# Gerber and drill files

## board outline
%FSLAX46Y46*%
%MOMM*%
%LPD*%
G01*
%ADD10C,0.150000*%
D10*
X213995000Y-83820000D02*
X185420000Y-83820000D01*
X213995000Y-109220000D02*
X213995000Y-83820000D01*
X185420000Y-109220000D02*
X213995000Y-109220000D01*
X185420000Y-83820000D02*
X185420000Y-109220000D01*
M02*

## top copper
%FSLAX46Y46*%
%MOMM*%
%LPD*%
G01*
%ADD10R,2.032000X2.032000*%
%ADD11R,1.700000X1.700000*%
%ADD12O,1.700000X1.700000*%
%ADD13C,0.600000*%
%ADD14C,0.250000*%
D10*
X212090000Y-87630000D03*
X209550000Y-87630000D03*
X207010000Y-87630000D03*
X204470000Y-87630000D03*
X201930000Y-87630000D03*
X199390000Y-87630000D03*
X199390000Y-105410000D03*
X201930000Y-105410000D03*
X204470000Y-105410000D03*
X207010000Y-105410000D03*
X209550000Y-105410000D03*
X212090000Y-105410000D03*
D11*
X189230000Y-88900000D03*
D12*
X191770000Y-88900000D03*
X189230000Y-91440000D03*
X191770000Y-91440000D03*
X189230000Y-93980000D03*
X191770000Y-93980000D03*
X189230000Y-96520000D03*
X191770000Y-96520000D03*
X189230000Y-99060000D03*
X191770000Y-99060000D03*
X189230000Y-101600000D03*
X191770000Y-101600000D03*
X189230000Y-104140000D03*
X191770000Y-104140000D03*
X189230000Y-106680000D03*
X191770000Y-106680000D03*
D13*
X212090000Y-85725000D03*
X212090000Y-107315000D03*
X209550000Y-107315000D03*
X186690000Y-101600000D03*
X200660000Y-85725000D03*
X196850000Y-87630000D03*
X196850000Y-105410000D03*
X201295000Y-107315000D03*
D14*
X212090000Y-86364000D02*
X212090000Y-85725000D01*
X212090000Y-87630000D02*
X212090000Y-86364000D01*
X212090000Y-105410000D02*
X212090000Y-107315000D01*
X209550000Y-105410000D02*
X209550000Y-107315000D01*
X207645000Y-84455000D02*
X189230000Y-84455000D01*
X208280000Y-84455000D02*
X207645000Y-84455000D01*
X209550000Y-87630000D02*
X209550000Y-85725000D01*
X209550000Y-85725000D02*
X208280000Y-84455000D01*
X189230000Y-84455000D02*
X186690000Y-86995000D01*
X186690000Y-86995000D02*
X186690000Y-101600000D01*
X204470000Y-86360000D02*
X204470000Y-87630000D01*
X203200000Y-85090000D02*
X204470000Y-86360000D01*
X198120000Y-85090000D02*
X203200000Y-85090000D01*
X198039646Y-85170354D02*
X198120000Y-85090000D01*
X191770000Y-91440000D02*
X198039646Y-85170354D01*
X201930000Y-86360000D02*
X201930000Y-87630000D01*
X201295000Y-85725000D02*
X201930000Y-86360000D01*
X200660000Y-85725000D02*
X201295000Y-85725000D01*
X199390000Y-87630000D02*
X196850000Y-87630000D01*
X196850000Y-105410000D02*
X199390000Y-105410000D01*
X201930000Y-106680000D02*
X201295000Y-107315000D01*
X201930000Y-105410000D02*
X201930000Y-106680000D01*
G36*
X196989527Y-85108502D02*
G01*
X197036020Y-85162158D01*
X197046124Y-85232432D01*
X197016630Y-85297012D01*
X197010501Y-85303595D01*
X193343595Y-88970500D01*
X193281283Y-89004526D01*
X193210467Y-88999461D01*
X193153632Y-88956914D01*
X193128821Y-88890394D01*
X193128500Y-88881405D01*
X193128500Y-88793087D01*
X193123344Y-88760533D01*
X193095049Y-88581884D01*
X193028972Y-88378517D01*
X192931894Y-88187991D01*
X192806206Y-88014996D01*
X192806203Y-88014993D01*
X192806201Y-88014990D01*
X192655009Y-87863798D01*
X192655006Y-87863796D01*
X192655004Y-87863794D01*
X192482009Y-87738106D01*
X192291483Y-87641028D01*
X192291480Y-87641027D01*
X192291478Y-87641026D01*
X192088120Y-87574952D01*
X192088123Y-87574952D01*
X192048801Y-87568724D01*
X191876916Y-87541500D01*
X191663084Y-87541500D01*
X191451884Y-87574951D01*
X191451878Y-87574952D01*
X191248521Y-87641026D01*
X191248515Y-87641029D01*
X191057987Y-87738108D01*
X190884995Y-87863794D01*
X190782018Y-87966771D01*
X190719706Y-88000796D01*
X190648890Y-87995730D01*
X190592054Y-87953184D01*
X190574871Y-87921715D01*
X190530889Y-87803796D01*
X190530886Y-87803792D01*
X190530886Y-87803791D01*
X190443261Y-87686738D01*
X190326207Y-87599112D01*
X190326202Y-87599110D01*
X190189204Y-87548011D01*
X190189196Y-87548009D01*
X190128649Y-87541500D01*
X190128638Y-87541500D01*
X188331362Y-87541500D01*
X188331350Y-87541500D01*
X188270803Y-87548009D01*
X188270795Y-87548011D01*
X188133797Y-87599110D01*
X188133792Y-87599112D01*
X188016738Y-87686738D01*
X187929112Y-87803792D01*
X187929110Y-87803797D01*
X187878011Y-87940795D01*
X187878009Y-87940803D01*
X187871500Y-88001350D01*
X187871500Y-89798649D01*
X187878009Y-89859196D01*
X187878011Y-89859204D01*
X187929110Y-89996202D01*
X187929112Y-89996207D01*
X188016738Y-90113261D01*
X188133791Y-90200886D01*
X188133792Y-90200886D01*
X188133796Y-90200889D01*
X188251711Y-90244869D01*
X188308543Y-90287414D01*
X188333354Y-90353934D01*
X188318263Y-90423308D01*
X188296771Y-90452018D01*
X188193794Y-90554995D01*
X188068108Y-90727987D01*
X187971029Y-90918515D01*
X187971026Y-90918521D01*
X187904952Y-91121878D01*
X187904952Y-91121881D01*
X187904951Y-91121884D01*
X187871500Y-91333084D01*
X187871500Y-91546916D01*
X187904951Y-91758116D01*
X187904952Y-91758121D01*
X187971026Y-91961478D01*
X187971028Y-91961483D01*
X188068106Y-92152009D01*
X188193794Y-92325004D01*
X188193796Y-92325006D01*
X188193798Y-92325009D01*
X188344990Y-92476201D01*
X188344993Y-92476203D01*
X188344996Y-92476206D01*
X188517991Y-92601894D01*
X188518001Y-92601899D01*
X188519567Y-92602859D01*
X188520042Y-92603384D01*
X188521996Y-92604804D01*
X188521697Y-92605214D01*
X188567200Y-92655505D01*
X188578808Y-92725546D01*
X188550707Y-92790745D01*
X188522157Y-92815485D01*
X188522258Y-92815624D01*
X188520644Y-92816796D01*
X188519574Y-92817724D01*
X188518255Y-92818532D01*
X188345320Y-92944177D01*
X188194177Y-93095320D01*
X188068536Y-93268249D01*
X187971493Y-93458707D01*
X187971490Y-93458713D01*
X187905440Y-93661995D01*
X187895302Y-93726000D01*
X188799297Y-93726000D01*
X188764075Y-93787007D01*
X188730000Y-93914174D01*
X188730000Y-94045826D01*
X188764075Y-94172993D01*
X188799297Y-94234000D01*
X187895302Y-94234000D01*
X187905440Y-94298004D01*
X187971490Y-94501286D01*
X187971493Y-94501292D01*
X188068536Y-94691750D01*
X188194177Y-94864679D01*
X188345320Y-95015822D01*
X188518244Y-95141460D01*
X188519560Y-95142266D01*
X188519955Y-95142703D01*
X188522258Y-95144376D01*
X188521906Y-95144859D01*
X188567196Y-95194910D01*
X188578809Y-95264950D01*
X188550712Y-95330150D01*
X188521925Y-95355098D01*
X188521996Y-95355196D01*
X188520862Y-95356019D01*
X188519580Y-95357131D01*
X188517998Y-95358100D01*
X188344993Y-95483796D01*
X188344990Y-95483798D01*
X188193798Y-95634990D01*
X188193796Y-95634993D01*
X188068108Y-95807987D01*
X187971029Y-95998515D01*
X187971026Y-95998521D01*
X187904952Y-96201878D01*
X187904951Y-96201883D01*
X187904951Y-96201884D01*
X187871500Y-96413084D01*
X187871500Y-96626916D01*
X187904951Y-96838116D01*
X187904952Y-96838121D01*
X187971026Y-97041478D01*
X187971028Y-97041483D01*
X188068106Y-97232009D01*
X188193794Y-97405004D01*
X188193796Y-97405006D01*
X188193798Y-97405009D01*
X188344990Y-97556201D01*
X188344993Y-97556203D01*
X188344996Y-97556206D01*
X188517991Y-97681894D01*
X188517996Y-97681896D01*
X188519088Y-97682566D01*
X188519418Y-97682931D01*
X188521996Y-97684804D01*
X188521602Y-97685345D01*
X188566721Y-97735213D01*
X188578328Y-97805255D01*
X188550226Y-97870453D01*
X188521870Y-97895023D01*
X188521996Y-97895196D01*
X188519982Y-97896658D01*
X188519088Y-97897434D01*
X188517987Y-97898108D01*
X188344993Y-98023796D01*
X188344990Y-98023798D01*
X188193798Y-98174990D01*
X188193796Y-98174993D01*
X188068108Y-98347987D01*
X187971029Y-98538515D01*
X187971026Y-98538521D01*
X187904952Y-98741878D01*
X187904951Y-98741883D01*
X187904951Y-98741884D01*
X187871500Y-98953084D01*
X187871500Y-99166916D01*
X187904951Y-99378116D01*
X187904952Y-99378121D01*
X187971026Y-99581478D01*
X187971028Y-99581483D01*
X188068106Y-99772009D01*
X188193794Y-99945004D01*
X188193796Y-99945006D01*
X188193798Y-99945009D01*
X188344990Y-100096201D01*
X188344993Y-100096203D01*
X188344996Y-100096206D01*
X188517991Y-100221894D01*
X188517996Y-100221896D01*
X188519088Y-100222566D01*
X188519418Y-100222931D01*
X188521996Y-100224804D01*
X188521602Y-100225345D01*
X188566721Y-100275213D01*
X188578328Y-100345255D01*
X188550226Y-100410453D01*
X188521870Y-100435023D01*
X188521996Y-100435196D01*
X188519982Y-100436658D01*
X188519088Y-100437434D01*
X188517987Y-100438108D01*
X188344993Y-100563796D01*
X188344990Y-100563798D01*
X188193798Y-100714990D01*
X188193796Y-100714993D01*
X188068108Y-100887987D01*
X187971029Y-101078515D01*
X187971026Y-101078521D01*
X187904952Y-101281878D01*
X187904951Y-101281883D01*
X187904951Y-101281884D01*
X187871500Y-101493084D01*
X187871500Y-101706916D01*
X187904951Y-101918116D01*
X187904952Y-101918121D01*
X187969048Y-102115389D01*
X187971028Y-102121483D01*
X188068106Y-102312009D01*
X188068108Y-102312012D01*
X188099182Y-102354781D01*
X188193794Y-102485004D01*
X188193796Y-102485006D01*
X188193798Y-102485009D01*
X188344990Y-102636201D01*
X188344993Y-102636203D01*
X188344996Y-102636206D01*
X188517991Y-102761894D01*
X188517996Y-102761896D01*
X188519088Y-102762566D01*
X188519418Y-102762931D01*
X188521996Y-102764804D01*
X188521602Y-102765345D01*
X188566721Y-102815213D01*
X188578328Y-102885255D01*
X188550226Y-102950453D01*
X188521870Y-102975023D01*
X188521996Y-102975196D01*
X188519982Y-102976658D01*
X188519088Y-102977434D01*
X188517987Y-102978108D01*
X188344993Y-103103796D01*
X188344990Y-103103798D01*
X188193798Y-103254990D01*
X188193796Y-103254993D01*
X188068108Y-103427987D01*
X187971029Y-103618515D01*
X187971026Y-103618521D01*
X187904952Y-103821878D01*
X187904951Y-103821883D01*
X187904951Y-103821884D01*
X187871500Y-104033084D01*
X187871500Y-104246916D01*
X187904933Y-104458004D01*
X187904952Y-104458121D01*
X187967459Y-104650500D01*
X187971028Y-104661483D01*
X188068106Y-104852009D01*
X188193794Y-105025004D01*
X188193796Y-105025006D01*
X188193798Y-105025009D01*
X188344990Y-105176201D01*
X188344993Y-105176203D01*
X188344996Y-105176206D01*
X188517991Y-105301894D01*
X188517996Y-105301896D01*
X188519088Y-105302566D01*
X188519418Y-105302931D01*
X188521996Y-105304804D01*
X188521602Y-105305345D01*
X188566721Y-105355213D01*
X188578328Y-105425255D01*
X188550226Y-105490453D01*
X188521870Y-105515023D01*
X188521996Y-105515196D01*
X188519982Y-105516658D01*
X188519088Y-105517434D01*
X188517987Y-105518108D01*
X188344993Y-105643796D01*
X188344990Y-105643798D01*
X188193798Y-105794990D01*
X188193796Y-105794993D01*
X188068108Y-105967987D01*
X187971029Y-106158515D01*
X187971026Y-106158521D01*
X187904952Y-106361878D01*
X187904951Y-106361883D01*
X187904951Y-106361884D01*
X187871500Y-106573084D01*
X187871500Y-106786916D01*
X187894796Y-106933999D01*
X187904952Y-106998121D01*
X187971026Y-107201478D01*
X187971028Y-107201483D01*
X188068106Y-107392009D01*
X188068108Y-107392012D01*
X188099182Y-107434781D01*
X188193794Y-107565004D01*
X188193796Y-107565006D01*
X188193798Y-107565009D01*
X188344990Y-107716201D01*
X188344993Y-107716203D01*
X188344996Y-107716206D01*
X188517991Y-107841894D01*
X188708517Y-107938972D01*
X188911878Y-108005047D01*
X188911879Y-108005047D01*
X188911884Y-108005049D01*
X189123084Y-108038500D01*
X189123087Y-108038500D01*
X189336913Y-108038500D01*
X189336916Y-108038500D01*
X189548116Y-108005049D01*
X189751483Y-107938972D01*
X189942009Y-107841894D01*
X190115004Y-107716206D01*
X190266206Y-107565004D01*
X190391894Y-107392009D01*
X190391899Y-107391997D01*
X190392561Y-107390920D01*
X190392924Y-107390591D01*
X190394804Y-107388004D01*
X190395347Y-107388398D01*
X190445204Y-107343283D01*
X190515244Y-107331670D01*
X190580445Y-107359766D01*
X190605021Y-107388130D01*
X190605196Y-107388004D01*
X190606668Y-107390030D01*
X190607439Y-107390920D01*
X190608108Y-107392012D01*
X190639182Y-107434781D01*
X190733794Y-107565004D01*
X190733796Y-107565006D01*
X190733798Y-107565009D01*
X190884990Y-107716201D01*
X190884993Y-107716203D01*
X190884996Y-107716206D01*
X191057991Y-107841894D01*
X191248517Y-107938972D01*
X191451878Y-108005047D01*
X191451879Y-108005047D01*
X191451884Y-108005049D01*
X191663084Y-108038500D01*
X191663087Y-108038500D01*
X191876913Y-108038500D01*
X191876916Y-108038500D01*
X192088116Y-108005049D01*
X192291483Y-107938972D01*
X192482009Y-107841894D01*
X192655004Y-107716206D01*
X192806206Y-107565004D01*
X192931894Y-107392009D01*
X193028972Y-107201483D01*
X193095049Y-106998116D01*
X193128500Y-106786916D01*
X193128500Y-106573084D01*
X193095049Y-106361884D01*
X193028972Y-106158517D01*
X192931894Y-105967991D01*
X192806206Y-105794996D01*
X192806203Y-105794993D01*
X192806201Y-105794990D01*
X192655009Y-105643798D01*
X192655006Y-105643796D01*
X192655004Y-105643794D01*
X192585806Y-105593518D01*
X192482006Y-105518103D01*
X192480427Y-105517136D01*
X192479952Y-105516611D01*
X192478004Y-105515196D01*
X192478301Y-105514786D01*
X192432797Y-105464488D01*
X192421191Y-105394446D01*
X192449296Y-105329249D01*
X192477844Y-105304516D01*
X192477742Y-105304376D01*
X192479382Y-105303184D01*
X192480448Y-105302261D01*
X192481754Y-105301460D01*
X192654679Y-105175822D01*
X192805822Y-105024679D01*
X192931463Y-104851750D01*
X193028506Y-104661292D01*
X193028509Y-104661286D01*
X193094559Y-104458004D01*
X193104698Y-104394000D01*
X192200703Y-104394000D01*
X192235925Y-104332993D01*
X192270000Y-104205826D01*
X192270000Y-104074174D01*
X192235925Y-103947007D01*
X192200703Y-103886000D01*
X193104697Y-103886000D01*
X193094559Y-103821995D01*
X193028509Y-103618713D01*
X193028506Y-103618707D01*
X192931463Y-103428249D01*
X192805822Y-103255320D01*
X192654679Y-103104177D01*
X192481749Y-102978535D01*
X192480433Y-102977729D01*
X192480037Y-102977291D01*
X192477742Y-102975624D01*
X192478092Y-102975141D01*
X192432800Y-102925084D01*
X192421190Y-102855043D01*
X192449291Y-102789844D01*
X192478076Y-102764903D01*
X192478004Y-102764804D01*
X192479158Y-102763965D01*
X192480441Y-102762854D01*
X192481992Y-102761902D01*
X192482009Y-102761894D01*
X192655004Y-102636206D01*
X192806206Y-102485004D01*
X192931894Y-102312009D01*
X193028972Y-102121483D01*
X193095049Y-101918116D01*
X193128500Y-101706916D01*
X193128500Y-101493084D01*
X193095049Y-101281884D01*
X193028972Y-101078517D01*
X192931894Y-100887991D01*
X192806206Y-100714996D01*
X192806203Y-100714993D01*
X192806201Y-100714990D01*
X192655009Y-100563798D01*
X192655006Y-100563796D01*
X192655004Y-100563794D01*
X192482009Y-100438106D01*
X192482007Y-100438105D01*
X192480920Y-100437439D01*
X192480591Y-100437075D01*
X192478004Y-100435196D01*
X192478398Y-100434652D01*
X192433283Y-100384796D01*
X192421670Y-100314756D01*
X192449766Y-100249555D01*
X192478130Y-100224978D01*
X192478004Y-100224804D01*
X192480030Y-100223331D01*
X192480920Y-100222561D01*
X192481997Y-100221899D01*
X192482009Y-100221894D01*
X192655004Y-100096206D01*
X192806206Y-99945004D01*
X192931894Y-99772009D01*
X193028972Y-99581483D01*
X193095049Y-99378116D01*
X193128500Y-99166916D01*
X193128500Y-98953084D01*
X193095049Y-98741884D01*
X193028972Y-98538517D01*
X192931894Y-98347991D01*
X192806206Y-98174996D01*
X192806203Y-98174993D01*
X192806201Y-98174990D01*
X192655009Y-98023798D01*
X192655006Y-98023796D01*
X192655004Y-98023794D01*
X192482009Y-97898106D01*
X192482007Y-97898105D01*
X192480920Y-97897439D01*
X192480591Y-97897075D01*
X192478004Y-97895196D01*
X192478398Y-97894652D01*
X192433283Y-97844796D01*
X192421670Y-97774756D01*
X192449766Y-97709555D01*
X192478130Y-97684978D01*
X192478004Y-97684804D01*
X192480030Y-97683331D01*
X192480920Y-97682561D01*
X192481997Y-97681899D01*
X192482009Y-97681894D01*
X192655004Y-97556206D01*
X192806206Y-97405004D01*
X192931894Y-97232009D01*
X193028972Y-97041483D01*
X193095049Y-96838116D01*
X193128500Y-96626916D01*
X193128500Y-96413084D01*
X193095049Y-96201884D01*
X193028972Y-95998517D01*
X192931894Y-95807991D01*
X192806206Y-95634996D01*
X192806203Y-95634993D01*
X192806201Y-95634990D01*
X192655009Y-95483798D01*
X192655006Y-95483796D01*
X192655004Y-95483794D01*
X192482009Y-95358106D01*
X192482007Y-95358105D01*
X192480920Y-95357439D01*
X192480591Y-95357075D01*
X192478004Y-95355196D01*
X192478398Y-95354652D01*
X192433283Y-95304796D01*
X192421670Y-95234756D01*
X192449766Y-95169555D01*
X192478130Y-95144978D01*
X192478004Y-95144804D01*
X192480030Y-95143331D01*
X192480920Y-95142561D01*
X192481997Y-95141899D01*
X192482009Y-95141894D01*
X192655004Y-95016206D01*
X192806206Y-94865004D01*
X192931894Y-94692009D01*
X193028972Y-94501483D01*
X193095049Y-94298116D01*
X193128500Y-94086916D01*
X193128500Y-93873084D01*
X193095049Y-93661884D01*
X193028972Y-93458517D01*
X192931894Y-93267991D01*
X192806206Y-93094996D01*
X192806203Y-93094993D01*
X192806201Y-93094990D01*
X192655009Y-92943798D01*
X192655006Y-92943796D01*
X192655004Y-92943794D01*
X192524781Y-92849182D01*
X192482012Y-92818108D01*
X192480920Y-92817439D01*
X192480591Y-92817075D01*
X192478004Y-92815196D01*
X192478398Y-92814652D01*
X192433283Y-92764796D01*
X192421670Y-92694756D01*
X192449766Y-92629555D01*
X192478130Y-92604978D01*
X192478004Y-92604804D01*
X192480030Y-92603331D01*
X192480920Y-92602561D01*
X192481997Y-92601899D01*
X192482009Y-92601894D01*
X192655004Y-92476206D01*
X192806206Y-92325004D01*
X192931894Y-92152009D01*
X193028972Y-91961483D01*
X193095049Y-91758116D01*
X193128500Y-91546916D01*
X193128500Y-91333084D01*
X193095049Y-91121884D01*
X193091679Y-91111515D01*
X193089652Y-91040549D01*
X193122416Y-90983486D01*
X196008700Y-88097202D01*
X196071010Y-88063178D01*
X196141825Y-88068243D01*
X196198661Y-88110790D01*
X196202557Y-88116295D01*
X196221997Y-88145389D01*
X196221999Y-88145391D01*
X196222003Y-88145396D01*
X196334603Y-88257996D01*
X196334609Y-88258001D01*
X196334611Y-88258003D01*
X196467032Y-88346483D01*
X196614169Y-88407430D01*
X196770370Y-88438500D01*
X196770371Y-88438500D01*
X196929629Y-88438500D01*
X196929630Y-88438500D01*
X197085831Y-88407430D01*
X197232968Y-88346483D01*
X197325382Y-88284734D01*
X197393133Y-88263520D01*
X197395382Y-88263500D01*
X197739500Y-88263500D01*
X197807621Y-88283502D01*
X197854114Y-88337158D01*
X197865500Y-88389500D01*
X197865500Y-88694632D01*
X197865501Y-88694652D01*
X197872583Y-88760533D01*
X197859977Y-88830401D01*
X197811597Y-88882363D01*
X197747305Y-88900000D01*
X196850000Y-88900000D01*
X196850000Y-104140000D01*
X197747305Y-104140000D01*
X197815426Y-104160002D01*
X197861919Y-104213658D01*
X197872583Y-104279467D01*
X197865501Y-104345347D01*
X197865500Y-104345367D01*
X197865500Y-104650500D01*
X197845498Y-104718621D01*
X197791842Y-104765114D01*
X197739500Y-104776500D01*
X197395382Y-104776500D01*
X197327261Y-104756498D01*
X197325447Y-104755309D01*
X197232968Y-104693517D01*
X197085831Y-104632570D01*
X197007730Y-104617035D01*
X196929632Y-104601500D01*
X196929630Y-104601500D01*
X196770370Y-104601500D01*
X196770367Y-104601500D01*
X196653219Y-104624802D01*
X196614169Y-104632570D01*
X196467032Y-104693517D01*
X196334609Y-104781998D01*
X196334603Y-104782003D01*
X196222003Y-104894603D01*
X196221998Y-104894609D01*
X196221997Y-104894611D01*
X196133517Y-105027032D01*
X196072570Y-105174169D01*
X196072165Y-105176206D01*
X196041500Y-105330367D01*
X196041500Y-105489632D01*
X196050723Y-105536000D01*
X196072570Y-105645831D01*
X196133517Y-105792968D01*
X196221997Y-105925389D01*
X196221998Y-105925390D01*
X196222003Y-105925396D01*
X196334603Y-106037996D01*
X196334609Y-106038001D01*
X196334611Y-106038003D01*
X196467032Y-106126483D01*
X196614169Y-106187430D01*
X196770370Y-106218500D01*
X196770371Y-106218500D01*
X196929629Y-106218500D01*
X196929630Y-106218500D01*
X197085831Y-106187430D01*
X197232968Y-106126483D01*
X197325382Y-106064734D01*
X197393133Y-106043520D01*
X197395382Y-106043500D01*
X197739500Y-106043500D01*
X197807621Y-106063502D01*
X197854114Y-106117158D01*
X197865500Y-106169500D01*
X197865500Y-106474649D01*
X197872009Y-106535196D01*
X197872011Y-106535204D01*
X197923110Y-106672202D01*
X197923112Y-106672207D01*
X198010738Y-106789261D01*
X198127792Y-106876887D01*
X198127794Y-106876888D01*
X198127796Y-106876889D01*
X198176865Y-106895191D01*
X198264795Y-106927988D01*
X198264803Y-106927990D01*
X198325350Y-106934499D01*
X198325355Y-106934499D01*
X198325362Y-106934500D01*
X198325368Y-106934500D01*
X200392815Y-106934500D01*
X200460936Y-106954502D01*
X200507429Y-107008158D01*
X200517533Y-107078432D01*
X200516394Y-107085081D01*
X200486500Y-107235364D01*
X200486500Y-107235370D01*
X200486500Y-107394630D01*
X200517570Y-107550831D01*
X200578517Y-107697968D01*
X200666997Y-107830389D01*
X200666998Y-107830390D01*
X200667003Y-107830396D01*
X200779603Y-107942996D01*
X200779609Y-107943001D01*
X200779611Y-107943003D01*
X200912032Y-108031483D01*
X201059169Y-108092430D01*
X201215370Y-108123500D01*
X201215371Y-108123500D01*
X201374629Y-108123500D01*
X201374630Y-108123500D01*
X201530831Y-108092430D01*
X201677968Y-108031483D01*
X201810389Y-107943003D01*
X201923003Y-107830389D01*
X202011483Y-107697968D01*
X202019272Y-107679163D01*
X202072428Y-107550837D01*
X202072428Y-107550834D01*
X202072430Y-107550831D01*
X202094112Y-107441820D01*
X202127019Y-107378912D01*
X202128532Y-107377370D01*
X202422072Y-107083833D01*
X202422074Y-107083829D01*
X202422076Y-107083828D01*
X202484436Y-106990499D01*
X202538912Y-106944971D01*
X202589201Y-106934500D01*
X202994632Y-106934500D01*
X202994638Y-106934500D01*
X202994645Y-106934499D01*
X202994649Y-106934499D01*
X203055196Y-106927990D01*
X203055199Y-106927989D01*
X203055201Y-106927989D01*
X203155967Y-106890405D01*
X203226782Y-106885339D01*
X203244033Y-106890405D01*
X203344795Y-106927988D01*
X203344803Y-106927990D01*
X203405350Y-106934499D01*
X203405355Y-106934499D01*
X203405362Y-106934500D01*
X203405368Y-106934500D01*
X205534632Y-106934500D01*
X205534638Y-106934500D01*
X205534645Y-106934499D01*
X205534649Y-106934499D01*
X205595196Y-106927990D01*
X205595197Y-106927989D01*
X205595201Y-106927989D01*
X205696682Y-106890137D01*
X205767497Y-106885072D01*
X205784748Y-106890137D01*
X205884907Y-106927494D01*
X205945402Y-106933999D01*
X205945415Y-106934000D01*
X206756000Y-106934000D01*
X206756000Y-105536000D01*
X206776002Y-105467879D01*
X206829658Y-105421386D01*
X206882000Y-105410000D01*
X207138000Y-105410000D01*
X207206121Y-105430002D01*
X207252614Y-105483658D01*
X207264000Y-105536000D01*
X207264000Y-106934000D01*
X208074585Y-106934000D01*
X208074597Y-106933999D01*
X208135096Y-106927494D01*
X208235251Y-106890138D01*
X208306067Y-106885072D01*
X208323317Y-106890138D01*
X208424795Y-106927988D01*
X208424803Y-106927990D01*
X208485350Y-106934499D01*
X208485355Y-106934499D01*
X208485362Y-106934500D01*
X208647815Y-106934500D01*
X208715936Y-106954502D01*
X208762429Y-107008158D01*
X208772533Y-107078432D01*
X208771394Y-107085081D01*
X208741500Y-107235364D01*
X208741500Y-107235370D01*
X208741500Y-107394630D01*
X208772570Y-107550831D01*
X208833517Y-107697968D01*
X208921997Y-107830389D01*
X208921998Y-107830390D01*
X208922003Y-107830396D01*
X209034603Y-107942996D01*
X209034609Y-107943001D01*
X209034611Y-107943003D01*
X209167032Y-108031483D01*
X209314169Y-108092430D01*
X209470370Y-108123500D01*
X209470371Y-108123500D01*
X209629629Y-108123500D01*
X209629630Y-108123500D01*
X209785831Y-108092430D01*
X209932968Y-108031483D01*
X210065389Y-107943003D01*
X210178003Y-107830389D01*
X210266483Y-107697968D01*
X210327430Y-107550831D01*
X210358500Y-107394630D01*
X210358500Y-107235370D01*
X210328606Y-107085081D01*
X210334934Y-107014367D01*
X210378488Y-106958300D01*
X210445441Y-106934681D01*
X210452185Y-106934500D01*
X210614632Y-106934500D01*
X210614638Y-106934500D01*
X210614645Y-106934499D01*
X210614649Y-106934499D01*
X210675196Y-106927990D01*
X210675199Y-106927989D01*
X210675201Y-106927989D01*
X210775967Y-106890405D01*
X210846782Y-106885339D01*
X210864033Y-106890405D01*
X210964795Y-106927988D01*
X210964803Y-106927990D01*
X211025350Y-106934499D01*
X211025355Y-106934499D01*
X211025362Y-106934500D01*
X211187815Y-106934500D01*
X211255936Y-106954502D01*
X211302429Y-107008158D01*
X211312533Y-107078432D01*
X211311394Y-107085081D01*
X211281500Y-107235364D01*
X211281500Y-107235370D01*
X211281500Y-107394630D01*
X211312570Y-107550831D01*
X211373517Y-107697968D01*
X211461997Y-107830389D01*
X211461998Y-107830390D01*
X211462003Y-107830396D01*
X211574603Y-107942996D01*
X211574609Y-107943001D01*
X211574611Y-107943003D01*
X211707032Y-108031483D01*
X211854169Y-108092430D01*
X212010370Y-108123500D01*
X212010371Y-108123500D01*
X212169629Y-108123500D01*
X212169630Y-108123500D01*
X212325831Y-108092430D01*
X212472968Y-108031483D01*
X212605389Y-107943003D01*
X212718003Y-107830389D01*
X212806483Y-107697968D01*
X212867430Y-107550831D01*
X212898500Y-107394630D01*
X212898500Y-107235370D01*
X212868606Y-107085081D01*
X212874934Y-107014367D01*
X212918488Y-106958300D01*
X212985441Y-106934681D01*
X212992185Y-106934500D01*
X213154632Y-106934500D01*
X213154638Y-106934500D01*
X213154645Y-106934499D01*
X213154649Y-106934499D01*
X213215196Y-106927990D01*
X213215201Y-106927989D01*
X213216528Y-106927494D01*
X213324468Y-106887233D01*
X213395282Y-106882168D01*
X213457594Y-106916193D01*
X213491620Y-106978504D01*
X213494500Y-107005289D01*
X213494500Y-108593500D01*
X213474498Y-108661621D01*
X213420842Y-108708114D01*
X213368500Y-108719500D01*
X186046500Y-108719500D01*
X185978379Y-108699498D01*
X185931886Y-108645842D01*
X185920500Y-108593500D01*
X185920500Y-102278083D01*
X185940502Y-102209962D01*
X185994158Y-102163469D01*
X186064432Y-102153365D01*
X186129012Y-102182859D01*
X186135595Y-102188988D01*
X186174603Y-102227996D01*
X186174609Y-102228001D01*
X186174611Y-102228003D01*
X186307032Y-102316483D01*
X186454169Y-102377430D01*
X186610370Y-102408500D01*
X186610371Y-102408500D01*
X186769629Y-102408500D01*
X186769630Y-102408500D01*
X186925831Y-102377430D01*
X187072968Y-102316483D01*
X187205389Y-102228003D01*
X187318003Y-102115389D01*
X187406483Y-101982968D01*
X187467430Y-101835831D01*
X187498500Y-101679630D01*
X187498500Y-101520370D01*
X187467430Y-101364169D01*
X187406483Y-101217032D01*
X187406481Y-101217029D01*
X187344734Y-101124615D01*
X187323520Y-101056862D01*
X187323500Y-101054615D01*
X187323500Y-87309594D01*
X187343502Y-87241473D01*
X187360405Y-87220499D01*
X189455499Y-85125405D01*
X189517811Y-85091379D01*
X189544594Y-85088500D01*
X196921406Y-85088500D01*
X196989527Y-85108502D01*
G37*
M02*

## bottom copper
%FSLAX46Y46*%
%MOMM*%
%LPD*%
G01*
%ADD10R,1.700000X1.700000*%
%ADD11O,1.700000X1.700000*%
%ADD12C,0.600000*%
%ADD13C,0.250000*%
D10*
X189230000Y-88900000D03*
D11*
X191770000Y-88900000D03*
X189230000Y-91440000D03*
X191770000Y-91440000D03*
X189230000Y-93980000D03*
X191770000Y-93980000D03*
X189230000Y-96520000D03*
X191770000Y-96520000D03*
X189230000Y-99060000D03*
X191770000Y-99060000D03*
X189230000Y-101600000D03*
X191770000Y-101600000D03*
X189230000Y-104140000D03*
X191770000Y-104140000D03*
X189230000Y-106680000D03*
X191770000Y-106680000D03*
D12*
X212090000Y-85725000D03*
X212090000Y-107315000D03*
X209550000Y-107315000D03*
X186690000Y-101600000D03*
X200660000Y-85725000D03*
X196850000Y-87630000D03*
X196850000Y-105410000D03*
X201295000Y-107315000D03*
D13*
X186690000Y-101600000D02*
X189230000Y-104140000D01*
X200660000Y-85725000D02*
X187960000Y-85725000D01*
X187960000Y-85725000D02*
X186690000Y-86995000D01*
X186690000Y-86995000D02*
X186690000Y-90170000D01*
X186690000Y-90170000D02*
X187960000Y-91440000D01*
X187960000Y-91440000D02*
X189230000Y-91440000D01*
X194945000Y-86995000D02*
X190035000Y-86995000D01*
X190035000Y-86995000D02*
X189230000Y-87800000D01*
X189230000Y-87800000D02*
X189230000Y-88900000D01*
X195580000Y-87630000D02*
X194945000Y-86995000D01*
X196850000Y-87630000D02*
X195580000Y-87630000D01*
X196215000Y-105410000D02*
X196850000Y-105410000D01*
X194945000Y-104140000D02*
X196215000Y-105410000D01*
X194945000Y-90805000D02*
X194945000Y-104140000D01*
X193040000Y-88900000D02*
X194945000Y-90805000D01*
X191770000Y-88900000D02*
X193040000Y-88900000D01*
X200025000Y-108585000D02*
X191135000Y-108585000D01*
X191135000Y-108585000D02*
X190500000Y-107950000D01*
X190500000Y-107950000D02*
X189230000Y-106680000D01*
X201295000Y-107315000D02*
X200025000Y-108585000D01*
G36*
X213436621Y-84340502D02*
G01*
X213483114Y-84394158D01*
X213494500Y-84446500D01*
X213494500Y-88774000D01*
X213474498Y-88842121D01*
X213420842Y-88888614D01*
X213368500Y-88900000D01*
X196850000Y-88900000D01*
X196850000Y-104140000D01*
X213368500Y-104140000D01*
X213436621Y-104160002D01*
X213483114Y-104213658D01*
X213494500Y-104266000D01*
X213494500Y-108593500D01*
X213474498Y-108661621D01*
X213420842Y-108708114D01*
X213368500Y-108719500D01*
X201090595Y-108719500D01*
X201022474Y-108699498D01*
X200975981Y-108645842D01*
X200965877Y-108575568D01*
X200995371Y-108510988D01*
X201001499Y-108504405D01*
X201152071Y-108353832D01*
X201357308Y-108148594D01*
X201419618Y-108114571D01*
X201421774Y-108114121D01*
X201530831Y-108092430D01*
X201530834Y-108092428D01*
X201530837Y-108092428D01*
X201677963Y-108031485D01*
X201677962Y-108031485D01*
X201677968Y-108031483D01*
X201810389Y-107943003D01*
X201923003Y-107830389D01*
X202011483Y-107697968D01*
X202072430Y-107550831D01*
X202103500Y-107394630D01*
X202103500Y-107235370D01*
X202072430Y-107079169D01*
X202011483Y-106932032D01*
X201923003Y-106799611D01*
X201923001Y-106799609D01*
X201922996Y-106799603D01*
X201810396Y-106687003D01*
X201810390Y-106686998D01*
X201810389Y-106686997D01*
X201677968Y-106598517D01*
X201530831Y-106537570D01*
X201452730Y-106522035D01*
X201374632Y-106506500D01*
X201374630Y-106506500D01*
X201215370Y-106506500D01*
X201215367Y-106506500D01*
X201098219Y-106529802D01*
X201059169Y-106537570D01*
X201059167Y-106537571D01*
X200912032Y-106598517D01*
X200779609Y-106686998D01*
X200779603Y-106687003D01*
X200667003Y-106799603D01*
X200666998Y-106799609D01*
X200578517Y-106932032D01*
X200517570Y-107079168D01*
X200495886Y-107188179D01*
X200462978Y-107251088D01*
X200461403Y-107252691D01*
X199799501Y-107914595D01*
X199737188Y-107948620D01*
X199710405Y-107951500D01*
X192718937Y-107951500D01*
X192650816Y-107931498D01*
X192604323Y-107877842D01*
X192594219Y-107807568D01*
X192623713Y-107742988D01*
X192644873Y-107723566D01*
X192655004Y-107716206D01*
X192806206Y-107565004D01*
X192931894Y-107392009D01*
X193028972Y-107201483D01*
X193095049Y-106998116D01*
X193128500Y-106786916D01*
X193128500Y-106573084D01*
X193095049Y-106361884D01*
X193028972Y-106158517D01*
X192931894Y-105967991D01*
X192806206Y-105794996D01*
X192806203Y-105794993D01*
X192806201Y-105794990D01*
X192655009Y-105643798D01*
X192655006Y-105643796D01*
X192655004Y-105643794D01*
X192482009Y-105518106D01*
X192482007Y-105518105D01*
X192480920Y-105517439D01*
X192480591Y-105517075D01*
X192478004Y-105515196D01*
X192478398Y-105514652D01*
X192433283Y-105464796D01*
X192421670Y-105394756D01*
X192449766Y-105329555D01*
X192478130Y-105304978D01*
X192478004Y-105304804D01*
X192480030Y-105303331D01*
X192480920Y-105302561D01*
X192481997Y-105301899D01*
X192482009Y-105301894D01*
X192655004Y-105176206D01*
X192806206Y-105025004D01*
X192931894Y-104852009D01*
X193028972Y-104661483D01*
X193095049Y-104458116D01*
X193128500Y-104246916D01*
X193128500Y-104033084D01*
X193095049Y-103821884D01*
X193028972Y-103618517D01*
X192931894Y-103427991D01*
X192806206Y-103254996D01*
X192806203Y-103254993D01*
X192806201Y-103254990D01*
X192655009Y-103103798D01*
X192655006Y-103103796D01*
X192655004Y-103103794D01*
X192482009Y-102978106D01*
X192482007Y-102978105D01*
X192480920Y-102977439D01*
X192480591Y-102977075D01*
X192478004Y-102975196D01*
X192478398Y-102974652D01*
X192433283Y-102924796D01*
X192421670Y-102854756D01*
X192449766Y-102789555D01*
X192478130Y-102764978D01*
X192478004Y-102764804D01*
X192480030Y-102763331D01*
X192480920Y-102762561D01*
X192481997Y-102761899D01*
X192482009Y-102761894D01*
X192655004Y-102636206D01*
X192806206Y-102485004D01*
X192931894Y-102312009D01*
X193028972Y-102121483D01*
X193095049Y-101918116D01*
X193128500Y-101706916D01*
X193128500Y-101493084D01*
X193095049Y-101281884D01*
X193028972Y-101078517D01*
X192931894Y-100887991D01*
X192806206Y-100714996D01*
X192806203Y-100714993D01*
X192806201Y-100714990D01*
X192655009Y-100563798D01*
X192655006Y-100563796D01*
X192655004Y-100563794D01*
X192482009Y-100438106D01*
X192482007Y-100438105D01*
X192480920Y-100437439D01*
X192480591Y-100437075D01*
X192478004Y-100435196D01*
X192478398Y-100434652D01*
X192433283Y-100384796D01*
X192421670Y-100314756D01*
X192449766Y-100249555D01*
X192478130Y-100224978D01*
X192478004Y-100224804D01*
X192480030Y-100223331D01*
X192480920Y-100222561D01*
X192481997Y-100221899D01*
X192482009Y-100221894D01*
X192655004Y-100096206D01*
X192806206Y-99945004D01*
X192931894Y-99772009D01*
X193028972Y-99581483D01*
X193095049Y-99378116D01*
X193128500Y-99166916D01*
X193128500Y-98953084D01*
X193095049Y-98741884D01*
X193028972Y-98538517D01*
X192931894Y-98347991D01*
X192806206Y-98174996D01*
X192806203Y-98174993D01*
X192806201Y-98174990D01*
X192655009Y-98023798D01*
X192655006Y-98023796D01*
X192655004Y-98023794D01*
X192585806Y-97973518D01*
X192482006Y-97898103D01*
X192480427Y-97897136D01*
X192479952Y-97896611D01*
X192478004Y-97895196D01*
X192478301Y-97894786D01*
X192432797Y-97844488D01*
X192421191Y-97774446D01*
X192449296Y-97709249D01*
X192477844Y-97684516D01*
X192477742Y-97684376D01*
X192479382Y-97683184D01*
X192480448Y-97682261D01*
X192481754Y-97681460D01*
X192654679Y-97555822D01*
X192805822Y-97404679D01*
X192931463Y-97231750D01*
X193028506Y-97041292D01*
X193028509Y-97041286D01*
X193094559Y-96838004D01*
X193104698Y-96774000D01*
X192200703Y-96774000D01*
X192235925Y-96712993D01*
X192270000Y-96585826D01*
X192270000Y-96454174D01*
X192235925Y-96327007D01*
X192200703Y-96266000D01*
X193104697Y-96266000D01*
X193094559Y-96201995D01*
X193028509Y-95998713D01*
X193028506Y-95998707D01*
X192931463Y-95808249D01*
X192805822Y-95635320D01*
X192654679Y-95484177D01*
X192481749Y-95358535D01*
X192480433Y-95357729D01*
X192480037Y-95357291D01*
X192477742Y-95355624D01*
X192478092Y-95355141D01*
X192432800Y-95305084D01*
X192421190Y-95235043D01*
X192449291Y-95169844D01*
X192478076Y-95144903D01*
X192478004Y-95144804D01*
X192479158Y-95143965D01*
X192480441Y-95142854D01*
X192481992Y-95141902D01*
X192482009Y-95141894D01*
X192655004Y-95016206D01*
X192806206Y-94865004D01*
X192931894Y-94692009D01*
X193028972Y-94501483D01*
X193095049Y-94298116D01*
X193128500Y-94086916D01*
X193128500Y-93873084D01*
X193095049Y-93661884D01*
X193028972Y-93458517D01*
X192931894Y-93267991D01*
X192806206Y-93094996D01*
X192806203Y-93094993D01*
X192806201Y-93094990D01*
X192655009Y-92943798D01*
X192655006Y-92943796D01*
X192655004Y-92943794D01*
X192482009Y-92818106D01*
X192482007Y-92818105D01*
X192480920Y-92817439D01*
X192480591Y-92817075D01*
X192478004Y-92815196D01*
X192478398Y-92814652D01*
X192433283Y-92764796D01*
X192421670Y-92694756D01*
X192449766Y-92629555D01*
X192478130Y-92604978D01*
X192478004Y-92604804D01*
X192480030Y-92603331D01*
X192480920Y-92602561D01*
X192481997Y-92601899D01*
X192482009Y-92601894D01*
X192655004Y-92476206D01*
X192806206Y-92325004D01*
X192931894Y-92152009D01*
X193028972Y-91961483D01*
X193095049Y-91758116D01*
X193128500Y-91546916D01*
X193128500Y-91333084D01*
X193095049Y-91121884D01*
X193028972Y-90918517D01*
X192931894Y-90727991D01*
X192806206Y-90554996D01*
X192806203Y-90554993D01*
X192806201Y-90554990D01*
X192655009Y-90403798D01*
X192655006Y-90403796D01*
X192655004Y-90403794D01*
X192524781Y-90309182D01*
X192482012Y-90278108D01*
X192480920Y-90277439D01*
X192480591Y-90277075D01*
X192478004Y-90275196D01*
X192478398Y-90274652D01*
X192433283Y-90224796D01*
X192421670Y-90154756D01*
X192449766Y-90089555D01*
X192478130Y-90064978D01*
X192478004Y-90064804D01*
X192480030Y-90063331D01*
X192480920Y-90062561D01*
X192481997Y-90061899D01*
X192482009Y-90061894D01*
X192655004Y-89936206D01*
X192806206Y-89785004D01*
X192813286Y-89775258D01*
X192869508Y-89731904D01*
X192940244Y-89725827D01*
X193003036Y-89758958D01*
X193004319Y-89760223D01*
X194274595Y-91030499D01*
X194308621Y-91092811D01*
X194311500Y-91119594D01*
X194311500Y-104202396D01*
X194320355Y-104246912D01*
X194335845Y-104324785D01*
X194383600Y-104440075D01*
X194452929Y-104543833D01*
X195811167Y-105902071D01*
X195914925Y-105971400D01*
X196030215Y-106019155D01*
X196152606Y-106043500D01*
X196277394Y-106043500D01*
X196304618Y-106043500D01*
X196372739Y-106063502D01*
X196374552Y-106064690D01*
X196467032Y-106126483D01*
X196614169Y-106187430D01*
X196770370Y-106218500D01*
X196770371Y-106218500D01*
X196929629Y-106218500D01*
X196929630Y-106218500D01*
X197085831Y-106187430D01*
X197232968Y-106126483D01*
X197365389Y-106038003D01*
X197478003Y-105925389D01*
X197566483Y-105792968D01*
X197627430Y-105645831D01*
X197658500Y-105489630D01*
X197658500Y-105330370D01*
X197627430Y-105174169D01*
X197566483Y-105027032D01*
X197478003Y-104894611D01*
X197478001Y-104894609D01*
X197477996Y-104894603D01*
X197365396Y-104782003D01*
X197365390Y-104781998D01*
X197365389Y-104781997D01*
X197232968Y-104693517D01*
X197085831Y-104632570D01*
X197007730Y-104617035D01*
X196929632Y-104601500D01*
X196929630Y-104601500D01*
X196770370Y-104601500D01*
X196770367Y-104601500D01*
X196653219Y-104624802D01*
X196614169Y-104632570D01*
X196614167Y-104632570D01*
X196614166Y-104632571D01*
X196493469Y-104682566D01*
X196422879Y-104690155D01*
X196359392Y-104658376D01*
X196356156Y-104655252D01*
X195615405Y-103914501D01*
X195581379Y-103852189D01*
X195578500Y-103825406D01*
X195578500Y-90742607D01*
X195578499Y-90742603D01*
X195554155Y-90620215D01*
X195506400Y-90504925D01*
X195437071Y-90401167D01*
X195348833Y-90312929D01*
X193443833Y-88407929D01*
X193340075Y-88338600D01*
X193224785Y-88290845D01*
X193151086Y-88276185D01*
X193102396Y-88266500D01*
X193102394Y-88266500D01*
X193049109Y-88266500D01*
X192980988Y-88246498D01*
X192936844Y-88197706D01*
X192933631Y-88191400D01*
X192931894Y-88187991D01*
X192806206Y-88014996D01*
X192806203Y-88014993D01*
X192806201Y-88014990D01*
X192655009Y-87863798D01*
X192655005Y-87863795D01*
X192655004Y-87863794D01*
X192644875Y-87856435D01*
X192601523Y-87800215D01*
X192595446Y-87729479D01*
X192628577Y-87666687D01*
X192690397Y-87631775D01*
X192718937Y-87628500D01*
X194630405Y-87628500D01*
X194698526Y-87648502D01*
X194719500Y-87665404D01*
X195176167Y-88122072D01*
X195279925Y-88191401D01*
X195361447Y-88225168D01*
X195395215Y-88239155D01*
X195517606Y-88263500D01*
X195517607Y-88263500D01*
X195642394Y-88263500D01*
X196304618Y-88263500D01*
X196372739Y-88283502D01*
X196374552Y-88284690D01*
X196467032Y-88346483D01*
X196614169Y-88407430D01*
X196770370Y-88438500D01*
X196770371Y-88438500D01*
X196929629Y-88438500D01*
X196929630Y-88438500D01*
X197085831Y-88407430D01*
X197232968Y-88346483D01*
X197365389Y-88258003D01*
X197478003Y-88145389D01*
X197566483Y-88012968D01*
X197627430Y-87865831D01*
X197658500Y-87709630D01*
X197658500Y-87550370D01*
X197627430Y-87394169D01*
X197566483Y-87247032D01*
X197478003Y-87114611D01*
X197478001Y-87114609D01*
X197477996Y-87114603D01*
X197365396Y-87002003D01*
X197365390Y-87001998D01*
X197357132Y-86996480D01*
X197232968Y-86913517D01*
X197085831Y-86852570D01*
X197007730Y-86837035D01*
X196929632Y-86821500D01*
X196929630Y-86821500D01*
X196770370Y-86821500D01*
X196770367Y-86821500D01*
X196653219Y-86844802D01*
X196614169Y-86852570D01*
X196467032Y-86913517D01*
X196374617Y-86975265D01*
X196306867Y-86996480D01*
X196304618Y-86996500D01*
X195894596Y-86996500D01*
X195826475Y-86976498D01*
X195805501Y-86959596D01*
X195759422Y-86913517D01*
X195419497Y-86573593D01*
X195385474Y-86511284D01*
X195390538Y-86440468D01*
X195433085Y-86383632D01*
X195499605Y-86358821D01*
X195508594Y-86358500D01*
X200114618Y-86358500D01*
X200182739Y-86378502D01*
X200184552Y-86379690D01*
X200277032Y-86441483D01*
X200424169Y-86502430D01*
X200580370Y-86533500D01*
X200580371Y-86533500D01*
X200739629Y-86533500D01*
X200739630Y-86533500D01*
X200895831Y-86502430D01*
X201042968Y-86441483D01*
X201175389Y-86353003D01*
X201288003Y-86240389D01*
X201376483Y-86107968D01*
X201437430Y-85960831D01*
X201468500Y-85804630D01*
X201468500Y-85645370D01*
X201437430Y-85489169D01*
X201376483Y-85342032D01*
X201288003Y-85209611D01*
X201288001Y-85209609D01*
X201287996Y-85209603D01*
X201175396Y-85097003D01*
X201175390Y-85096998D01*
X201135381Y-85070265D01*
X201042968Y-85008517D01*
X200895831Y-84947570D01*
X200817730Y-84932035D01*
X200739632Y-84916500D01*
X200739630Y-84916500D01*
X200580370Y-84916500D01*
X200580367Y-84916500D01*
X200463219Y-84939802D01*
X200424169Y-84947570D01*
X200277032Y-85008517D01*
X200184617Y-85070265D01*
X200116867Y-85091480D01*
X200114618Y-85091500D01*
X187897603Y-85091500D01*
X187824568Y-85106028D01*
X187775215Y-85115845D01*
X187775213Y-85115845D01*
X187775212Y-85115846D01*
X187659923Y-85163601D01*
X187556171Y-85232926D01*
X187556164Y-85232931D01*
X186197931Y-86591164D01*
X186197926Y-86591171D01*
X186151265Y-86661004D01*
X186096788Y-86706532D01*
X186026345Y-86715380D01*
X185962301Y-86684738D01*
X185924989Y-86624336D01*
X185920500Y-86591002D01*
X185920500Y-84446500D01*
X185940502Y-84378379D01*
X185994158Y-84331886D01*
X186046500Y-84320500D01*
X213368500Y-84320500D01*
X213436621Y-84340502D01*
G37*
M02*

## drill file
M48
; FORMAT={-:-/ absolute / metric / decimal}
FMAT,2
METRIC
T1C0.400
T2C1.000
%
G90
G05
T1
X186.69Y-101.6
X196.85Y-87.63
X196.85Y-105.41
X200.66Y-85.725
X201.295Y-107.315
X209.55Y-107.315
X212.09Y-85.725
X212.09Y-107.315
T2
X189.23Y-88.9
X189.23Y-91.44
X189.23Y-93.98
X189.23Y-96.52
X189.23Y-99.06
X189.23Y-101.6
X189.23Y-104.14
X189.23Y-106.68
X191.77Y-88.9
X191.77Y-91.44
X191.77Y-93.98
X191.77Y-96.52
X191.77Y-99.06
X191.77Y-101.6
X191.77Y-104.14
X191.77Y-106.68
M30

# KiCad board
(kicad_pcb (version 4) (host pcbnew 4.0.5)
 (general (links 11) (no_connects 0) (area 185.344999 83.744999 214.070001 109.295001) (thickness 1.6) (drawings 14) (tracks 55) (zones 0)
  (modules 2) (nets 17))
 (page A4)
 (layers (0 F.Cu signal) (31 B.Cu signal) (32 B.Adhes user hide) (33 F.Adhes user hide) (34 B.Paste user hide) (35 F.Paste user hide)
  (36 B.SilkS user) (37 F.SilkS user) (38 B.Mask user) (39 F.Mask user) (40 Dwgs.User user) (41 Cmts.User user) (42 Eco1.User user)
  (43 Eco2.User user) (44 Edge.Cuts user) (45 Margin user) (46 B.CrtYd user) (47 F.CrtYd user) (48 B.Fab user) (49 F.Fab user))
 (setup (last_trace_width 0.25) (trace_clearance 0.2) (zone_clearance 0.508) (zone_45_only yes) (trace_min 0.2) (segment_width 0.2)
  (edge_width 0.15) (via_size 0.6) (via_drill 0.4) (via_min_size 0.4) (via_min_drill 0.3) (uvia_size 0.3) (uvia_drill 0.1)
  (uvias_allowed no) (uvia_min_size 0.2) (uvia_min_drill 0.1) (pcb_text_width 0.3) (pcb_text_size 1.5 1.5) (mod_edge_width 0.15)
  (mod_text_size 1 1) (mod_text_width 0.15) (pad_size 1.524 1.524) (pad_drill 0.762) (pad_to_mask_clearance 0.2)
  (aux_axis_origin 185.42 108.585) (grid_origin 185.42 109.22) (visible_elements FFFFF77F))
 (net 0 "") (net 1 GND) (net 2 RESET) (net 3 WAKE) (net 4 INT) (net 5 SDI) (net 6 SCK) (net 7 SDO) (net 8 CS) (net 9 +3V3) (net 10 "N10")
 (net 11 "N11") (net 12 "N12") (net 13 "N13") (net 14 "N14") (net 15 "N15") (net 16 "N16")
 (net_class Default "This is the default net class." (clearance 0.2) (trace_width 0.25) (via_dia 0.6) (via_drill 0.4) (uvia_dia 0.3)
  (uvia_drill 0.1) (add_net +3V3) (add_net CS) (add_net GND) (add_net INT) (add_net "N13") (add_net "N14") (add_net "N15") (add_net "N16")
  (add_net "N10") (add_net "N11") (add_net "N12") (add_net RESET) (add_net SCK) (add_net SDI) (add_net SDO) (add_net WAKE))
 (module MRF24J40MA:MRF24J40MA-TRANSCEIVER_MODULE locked (layer F.Cu) (at 197.866 87.63 270)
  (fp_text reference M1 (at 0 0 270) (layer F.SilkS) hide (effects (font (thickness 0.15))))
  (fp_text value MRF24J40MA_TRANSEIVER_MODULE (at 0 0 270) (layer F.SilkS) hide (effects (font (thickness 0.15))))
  (pad 1 smd rect (at 0 -14.224 270) (size 2.032 2.032) (layers F.Cu F.Paste F.Mask) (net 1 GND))
  (pad 2 smd rect (at 0 -11.684 270) (size 2.032 2.032) (layers F.Cu F.Paste F.Mask) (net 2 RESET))
  (pad 3 smd rect (at 0 -9.144 270) (size 2.032 2.032) (layers F.Cu F.Paste F.Mask) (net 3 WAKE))
  (pad 4 smd rect (at 0 -6.604 270) (size 2.032 2.032) (layers F.Cu F.Paste F.Mask) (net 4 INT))
  (pad 5 smd rect (at 0 -4.064 270) (size 2.032 2.032) (layers F.Cu F.Paste F.Mask) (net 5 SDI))
  (pad 6 smd rect (at 0 -1.524 270) (size 2.032 2.032) (layers F.Cu F.Paste F.Mask) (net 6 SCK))
  (pad 7 smd rect (at 17.78 -1.524 270) (size 2.032 2.032) (layers F.Cu F.Paste F.Mask) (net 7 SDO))
  (pad 8 smd rect (at 17.78 -4.064 270) (size 2.032 2.032) (layers F.Cu F.Paste F.Mask) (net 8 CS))
  (pad 9 smd rect (at 17.78 -6.604 270) (size 2.032 2.032) (layers F.Cu F.Paste F.Mask))
  (pad 10 smd rect (at 17.78 -9.144 270) (size 2.032 2.032) (layers F.Cu F.Paste F.Mask) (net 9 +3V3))
  (pad 11 smd rect (at 17.78 -11.684 270) (size 2.032 2.032) (layers F.Cu F.Paste F.Mask) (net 1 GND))
  (pad 12 smd rect (at 17.78 -14.224 270) (size 2.032 2.032) (layers F.Cu F.Paste F.Mask) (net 1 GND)))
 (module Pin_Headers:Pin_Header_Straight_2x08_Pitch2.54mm (layer F.Cu) (at 189.23 88.9)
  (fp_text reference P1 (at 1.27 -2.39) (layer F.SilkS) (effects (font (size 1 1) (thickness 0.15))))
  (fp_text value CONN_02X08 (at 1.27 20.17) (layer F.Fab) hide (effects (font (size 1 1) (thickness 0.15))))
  (pad 1 thru_hole rect (at 0 0) (size 1.7 1.7) (drill 1) (layers *.Cu *.Mask) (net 6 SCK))
  (pad 2 thru_hole oval (at 2.54 0) (size 1.7 1.7) (drill 1) (layers *.Cu *.Mask) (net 7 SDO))
  (pad 3 thru_hole oval (at 0 2.54) (size 1.7 1.7) (drill 1) (layers *.Cu *.Mask) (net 5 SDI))
  (pad 4 thru_hole oval (at 2.54 2.54) (size 1.7 1.7) (drill 1) (layers *.Cu *.Mask) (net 4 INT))
  (pad 5 thru_hole oval (at 0 5.08) (size 1.7 1.7) (drill 1) (layers *.Cu *.Mask) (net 9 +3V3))
  (pad 6 thru_hole oval (at 2.54 5.08) (size 1.7 1.7) (drill 1) (layers *.Cu *.Mask) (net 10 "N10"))
  (pad 7 thru_hole oval (at 0 7.62) (size 1.7 1.7) (drill 1) (layers *.Cu *.Mask) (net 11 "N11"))
  (pad 8 thru_hole oval (at 2.54 7.62) (size 1.7 1.7) (drill 1) (layers *.Cu *.Mask) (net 1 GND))
  (pad 9 thru_hole oval (at 0 10.16) (size 1.7 1.7) (drill 1) (layers *.Cu *.Mask) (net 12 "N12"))
  (pad 10 thru_hole oval (at 2.54 10.16) (size 1.7 1.7) (drill 1) (layers *.Cu *.Mask) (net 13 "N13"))
  (pad 11 thru_hole oval (at 0 12.7) (size 1.7 1.7) (drill 1) (layers *.Cu *.Mask) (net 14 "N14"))
  (pad 12 thru_hole oval (at 2.54 12.7) (size 1.7 1.7) (drill 1) (layers *.Cu *.Mask) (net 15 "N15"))
  (pad 13 thru_hole oval (at 0 15.24) (size 1.7 1.7) (drill 1) (layers *.Cu *.Mask) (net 2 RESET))
  (pad 14 thru_hole oval (at 2.54 15.24) (size 1.7 1.7) (drill 1) (layers *.Cu *.Mask) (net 9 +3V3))
  (pad 15 thru_hole oval (at 0 17.78) (size 1.7 1.7) (drill 1) (layers *.Cu *.Mask) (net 8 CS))
  (pad 16 thru_hole oval (at 2.54 17.78) (size 1.7 1.7) (drill 1) (layers *.Cu *.Mask) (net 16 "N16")))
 (gr_line (start 213.995 83.82) (end 185.42 83.82) (layer Edge.Cuts) (width 0.15))
 (gr_line (start 213.995 109.22) (end 213.995 83.82) (layer Edge.Cuts) (width 0.15))
 (gr_line (start 185.42 109.22) (end 213.995 109.22) (layer Edge.Cuts) (width 0.15))
 (gr_line (start 185.42 83.82) (end 185.42 109.22) (layer Edge.Cuts) (width 0.15))
 (segment (start 185.42 84.455) (end 184.785 84.455) (width 0.25) (layer Dwgs.User) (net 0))
 (segment (start 213.36 84.455) (end 185.42 84.455) (width 0.25) (layer Dwgs.User) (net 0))
 (segment (start 213.36 85.09) (end 213.36 84.455) (width 0.25) (layer Dwgs.User) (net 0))
 (segment (start 213.995 84.455) (end 213.36 85.09) (width 0.25) (layer Dwgs.User) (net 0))
 (segment (start 185.42 84.455) (end 213.995 84.455) (width 0.25) (layer Dwgs.User) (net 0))
 (segment (start 212.09 86.364) (end 212.09 85.725) (width 0.25) (layer F.Cu) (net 1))
 (via (at 212.09 85.725) (size 0.6) (drill 0.4) (layers F.Cu B.Cu) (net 1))
 (segment (start 212.09 87.63) (end 212.09 86.364) (width 0.25) (layer F.Cu) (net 1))
 (via (at 212.09 107.315) (size 0.6) (drill 0.4) (layers F.Cu B.Cu) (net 1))
 (segment (start 212.09 105.41) (end 212.09 107.315) (width 0.25) (layer F.Cu) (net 1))
 (via (at 209.55 107.315) (size 0.6) (drill 0.4) (layers F.Cu B.Cu) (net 1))
 (segment (start 209.55 105.41) (end 209.55 107.315) (width 0.25) (layer F.Cu) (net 1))
 (segment (start 186.69 101.6) (end 189.23 104.14) (width 0.25) (layer B.Cu) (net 2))
 (via (at 186.69 101.6) (size 0.6) (drill 0.4) (layers F.Cu B.Cu) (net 2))
 (segment (start 207.645 84.455) (end 189.23 84.455) (width 0.25) (layer F.Cu) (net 2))
 (segment (start 208.28 84.455) (end 207.645 84.455) (width 0.25) (layer F.Cu) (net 2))
 (segment (start 209.55 87.63) (end 209.55 85.725) (width 0.25) (layer F.Cu) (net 2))
 (segment (start 209.55 85.725) (end 208.28 84.455) (width 0.25) (layer F.Cu) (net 2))
 (segment (start 189.23 84.455) (end 186.69 86.995) (width 0.25) (layer F.Cu) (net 2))
 (segment (start 186.69 86.995) (end 186.69 101.6) (width 0.25) (layer F.Cu) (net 2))
 (segment (start 204.47 86.36) (end 204.47 87.63) (width 0.25) (layer F.Cu) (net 4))
 (segment (start 203.2 85.09) (end 204.47 86.36) (width 0.25) (layer F.Cu) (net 4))
 (segment (start 198.12 85.09) (end 203.2 85.09) (width 0.25) (layer F.Cu) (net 4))
 (segment (start 198.039646 85.170354) (end 198.12 85.09) (width 0.25) (layer F.Cu) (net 4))
 (segment (start 191.77 91.44) (end 198.039646 85.170354) (width 0.25) (layer F.Cu) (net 4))
 (segment (start 201.93 86.36) (end 201.93 87.63) (width 0.25) (layer F.Cu) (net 5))
 (segment (start 201.295 85.725) (end 201.93 86.36) (width 0.25) (layer F.Cu) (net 5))
 (segment (start 200.66 85.725) (end 201.295 85.725) (width 0.25) (layer F.Cu) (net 5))
 (via (at 200.66 85.725) (size 0.6) (drill 0.4) (layers F.Cu B.Cu) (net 5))
 (segment (start 200.66 85.725) (end 187.96 85.725) (width 0.25) (layer B.Cu) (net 5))
 (segment (start 187.96 85.725) (end 186.69 86.995) (width 0.25) (layer B.Cu) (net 5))
 (segment (start 186.69 86.995) (end 186.69 90.17) (width 0.25) (layer B.Cu) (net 5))
 (segment (start 186.69 90.17) (end 187.96 91.44) (width 0.25) (layer B.Cu) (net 5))
 (segment (start 187.96 91.44) (end 189.23 91.44) (width 0.25) (layer B.Cu) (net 5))
 (segment (start 194.945 86.995) (end 190.035 86.995) (width 0.25) (layer B.Cu) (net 6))
 (segment (start 190.035 86.995) (end 189.23 87.8) (width 0.25) (layer B.Cu) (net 6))
 (segment (start 189.23 87.8) (end 189.23 88.9) (width 0.25) (layer B.Cu) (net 6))
 (segment (start 195.58 87.63) (end 194.945 86.995) (width 0.25) (layer B.Cu) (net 6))
 (segment (start 196.85 87.63) (end 195.58 87.63) (width 0.25) (layer B.Cu) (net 6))
 (via (at 196.85 87.63) (size 0.6) (drill 0.4) (layers F.Cu B.Cu) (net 6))
 (segment (start 199.39 87.63) (end 196.85 87.63) (width 0.25) (layer F.Cu) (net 6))
 (segment (start 196.85 105.41) (end 199.39 105.41) (width 0.25) (layer F.Cu) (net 7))
 (segment (start 196.215 105.41) (end 196.85 105.41) (width 0.25) (layer B.Cu) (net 7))
 (via (at 196.85 105.41) (size 0.6) (drill 0.4) (layers F.Cu B.Cu) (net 7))
 (segment (start 194.945 104.14) (end 196.215 105.41) (width 0.25) (layer B.Cu) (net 7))
 (segment (start 194.945 90.805) (end 194.945 104.14) (width 0.25) (layer B.Cu) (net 7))
 (segment (start 193.04 88.9) (end 194.945 90.805) (width 0.25) (layer B.Cu) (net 7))
 (segment (start 191.77 88.9) (end 193.04 88.9) (width 0.25) (layer B.Cu) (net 7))
 (segment (start 200.025 108.585) (end 191.135 108.585) (width 0.25) (layer B.Cu) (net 8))
 (segment (start 191.135 108.585) (end 190.5 107.95) (width 0.25) (layer B.Cu) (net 8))
 (segment (start 190.5 107.95) (end 189.23 106.68) (width 0.25) (layer B.Cu) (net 8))
 (segment (start 201.295 107.315) (end 200.025 108.585) (width 0.25) (layer B.Cu) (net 8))
 (via (at 201.295 107.315) (size 0.6) (drill 0.4) (layers F.Cu B.Cu) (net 8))
 (segment (start 201.93 106.68) (end 201.295 107.315) (width 0.25) (layer F.Cu) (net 8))
 (segment (start 201.93 105.41) (end 201.93 106.68) (width 0.25) (layer F.Cu) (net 8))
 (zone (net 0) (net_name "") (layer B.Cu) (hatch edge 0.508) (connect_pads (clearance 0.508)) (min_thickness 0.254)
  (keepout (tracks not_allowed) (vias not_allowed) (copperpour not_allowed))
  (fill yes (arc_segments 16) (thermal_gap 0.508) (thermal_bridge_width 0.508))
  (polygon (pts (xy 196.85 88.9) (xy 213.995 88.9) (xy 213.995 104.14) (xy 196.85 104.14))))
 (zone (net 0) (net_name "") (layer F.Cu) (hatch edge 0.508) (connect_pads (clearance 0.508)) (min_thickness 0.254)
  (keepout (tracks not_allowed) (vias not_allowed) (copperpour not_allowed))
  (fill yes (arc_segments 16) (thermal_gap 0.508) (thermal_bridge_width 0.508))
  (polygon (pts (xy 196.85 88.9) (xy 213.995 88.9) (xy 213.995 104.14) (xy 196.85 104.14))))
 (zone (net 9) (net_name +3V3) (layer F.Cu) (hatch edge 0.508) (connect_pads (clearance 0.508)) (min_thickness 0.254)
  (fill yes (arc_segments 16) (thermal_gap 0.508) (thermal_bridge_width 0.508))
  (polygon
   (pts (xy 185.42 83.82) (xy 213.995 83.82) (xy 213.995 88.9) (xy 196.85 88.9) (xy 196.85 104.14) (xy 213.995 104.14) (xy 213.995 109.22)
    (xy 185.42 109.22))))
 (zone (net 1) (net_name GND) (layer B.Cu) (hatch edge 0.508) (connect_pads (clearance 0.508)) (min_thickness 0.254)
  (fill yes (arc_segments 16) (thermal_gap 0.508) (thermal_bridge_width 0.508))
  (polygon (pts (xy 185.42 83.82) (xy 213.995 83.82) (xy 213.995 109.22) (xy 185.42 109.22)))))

